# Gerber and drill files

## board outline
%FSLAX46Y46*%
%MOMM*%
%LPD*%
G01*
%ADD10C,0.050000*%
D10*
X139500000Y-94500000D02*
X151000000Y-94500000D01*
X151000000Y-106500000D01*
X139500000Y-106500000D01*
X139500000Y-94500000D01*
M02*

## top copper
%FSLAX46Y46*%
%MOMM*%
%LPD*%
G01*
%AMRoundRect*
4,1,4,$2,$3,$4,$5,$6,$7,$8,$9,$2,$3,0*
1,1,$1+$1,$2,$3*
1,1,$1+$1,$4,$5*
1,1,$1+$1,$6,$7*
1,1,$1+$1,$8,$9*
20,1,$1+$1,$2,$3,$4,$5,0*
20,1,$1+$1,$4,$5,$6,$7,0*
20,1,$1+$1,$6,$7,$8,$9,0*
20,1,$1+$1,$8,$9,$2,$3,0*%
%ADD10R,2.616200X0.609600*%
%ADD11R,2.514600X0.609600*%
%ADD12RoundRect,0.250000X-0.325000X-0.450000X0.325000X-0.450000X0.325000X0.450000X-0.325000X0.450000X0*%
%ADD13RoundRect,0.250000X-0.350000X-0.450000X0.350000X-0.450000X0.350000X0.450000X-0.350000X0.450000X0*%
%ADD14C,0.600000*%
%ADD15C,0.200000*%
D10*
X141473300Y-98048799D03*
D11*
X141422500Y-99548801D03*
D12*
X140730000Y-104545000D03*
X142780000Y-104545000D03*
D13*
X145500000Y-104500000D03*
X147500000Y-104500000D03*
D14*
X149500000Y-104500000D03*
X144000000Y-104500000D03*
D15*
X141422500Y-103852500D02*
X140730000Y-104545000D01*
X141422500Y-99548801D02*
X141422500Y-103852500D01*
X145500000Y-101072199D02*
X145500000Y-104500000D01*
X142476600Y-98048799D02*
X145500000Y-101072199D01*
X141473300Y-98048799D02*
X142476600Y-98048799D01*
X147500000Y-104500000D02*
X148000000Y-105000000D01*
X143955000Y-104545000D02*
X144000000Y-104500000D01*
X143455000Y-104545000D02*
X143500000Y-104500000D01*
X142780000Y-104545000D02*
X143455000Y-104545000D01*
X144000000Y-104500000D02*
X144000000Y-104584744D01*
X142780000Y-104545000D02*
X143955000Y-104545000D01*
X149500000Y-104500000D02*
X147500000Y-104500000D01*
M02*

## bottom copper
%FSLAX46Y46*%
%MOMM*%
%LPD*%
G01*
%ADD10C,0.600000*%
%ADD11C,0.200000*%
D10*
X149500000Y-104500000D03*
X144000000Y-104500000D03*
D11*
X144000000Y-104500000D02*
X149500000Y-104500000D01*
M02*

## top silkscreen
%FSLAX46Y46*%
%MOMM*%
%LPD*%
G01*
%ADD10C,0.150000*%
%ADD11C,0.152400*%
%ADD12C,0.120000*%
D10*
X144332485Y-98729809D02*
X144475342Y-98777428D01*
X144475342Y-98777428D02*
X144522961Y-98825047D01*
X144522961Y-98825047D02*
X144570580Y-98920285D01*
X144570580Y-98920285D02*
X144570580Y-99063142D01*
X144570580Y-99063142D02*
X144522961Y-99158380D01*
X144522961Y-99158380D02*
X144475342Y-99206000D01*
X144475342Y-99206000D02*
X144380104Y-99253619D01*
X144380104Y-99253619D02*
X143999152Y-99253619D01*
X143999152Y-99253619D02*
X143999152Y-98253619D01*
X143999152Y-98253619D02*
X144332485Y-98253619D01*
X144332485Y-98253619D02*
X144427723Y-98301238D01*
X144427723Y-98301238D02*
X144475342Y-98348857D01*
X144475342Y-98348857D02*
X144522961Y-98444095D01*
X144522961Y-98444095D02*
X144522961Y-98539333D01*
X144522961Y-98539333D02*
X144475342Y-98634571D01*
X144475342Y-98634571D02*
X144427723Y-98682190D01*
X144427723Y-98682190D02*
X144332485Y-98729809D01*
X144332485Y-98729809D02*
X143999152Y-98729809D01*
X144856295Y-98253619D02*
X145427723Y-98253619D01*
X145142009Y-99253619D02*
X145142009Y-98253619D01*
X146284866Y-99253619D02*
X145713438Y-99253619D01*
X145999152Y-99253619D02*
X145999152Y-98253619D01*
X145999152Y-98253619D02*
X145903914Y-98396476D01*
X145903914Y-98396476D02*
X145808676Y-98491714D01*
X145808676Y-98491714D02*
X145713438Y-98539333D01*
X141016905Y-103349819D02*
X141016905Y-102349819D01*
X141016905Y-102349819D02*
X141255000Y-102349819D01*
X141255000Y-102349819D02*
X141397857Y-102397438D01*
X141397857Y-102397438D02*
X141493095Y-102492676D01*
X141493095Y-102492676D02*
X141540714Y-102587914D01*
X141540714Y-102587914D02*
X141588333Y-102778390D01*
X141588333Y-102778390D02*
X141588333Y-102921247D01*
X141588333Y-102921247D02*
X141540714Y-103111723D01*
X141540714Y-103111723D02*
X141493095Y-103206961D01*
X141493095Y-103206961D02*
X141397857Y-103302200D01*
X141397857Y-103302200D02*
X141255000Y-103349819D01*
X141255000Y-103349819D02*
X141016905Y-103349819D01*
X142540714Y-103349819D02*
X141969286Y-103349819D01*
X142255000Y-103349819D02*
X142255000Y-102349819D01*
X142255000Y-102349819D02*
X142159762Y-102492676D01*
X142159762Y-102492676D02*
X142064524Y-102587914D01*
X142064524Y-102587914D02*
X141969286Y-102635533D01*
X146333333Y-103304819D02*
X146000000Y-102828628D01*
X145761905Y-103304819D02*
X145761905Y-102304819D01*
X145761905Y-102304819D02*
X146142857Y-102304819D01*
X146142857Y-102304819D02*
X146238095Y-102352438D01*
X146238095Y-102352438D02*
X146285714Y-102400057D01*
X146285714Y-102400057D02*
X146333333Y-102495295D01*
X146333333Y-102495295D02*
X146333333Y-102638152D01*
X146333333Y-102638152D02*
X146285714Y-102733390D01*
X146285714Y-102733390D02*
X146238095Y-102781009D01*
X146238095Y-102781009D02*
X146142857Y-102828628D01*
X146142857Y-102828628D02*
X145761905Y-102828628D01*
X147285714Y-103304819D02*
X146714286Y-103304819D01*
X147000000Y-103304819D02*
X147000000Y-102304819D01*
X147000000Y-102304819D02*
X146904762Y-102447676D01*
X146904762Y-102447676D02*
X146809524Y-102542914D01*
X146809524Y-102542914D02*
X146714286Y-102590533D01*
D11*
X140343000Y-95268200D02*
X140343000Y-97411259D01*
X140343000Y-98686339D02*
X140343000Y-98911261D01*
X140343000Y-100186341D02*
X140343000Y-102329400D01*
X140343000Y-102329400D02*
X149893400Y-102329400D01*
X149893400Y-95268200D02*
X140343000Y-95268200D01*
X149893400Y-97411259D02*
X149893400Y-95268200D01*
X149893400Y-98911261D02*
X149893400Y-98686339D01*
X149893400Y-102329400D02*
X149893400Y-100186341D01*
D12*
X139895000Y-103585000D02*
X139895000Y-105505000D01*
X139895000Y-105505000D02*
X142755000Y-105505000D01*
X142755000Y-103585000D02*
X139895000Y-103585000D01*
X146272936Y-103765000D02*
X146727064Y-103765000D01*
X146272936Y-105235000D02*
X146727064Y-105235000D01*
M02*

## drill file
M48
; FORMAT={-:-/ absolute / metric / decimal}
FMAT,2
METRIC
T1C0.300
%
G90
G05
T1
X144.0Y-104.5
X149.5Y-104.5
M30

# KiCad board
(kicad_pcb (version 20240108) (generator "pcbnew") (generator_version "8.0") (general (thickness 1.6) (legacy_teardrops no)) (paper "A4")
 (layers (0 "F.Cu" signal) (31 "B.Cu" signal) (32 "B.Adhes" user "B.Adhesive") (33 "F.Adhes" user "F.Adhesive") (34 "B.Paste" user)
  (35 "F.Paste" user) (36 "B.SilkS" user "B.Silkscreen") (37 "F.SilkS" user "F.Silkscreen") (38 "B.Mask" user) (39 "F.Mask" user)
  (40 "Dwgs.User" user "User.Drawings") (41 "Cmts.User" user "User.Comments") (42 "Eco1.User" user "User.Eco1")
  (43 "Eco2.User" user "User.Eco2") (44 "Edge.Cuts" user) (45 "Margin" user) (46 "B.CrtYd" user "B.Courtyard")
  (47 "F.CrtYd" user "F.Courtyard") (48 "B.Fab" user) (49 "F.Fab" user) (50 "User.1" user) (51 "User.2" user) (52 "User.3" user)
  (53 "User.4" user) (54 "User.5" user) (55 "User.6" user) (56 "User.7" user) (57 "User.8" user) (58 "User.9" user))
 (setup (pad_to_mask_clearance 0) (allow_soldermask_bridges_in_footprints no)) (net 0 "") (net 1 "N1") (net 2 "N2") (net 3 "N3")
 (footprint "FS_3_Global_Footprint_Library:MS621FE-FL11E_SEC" (layer "F.Cu") (at 145.1182 98.7988)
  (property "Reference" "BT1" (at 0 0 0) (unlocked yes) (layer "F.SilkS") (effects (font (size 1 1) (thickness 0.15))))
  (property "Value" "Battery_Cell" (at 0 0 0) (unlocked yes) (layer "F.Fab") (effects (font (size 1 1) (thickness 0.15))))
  (fp_line (start -4.7752 -3.5306) (end -4.7752 -1.387541) (stroke (width 0.1524) (type solid)) (layer "F.SilkS"))
  (fp_line (start -4.7752 -0.112461) (end -4.7752 0.112461) (stroke (width 0.1524) (type solid)) (layer "F.SilkS"))
  (fp_line (start -4.7752 1.387541) (end -4.7752 3.5306) (stroke (width 0.1524) (type solid)) (layer "F.SilkS"))
  (fp_line (start -4.7752 3.5306) (end 4.7752 3.5306) (stroke (width 0.1524) (type solid)) (layer "F.SilkS"))
  (fp_line (start 4.7752 -3.5306) (end -4.7752 -3.5306) (stroke (width 0.1524) (type solid)) (layer "F.SilkS"))
  (fp_line (start 4.7752 -1.387541) (end 4.7752 -3.5306) (stroke (width 0.1524) (type solid)) (layer "F.SilkS"))
  (fp_line (start 4.7752 0.112461) (end 4.7752 -0.112461) (stroke (width 0.1524) (type solid)) (layer "F.SilkS"))
  (fp_line (start 4.7752 3.5306) (end 4.7752 1.387541) (stroke (width 0.1524) (type solid)) (layer "F.SilkS"))
  (pad "1" smd rect (at -3.6449 -0.750001) (size 2.6162 0.6096) (layers "F.Cu" "F.Paste" "F.Mask") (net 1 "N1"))
  (pad "2" smd rect (at -3.6957 0.750001) (size 2.5146 0.6096) (layers "F.Cu" "F.Paste" "F.Mask") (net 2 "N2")))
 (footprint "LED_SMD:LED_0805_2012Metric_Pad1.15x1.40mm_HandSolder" (layer "F.Cu") (at 141.755 104.545)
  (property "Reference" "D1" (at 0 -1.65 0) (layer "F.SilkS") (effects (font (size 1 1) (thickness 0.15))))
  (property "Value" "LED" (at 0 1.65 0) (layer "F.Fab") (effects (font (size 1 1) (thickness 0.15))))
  (fp_line (start -1.86 -0.96) (end -1.86 0.96) (stroke (width 0.12) (type solid)) (layer "F.SilkS"))
  (fp_line (start -1.86 0.96) (end 1 0.96) (stroke (width 0.12) (type solid)) (layer "F.SilkS"))
  (fp_line (start 1 -0.96) (end -1.86 -0.96) (stroke (width 0.12) (type solid)) (layer "F.SilkS"))
  (pad "1" smd roundrect (at -1.025 0) (size 1.15 1.4) (layers "F.Cu" "F.Paste" "F.Mask") (roundrect_rratio 0.217391) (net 2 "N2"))
  (pad "2" smd roundrect (at 1.025 0) (size 1.15 1.4) (layers "F.Cu" "F.Paste" "F.Mask") (roundrect_rratio 0.217391) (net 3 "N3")))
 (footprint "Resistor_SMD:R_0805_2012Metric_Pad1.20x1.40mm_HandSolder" (layer "F.Cu") (at 146.5 104.5)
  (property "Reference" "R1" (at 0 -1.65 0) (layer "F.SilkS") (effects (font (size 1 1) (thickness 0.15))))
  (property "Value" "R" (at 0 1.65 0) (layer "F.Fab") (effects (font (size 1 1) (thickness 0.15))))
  (fp_line (start -0.227064 -0.735) (end 0.227064 -0.735) (stroke (width 0.12) (type solid)) (layer "F.SilkS"))
  (fp_line (start -0.227064 0.735) (end 0.227064 0.735) (stroke (width 0.12) (type solid)) (layer "F.SilkS"))
  (pad "1" smd roundrect (at -1 0) (size 1.2 1.4) (layers "F.Cu" "F.Paste" "F.Mask") (roundrect_rratio 0.208333) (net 1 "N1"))
  (pad "2" smd roundrect (at 1 0) (size 1.2 1.4) (layers "F.Cu" "F.Paste" "F.Mask") (roundrect_rratio 0.208333) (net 3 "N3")))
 (gr_rect (start 139.5 94.5) (end 151 106.5) (stroke (width 0.05) (type default)) (fill none) (layer "Edge.Cuts"))
 (segment (start 141.4225 103.8525) (end 140.73 104.545) (width 0.2) (layer "F.Cu") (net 2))
 (segment (start 141.4225 99.548801) (end 141.4225 103.8525) (width 0.2) (layer "F.Cu") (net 2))
 (segment (start 145.5 101.072199) (end 145.5 104.5) (width 0.2) (layer "F.Cu") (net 1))
 (segment (start 142.4766 98.048799) (end 145.5 101.072199) (width 0.2) (layer "F.Cu") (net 1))
 (segment (start 141.4733 98.048799) (end 142.4766 98.048799) (width 0.2) (layer "F.Cu") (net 1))
 (segment (start 147.5 104.5) (end 148 105) (width 0.2) (layer "F.Cu") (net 3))
 (segment (start 143.955 104.545) (end 144 104.5) (width 0.2) (layer "F.Cu") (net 3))
 (segment (start 143.455 104.545) (end 143.5 104.5) (width 0.2) (layer "F.Cu") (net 3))
 (segment (start 142.78 104.545) (end 143.455 104.545) (width 0.2) (layer "F.Cu") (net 3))
 (segment (start 144 104.5) (end 144 104.584744) (width 0.2) (layer "F.Cu") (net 3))
 (segment (start 142.78 104.545) (end 143.955 104.545) (width 0.2) (layer "F.Cu") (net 3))
 (segment (start 149.5 104.5) (end 147.5 104.5) (width 0.2) (layer "F.Cu") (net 3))
 (via (at 149.5 104.5) (size 0.6) (drill 0.3) (layers "F.Cu" "B.Cu") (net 3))
 (via (at 144 104.5) (size 0.6) (drill 0.3) (layers "F.Cu" "B.Cu") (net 3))
 (segment (start 144 104.5) (end 149.5 104.5) (width 0.2) (layer "B.Cu") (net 3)))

